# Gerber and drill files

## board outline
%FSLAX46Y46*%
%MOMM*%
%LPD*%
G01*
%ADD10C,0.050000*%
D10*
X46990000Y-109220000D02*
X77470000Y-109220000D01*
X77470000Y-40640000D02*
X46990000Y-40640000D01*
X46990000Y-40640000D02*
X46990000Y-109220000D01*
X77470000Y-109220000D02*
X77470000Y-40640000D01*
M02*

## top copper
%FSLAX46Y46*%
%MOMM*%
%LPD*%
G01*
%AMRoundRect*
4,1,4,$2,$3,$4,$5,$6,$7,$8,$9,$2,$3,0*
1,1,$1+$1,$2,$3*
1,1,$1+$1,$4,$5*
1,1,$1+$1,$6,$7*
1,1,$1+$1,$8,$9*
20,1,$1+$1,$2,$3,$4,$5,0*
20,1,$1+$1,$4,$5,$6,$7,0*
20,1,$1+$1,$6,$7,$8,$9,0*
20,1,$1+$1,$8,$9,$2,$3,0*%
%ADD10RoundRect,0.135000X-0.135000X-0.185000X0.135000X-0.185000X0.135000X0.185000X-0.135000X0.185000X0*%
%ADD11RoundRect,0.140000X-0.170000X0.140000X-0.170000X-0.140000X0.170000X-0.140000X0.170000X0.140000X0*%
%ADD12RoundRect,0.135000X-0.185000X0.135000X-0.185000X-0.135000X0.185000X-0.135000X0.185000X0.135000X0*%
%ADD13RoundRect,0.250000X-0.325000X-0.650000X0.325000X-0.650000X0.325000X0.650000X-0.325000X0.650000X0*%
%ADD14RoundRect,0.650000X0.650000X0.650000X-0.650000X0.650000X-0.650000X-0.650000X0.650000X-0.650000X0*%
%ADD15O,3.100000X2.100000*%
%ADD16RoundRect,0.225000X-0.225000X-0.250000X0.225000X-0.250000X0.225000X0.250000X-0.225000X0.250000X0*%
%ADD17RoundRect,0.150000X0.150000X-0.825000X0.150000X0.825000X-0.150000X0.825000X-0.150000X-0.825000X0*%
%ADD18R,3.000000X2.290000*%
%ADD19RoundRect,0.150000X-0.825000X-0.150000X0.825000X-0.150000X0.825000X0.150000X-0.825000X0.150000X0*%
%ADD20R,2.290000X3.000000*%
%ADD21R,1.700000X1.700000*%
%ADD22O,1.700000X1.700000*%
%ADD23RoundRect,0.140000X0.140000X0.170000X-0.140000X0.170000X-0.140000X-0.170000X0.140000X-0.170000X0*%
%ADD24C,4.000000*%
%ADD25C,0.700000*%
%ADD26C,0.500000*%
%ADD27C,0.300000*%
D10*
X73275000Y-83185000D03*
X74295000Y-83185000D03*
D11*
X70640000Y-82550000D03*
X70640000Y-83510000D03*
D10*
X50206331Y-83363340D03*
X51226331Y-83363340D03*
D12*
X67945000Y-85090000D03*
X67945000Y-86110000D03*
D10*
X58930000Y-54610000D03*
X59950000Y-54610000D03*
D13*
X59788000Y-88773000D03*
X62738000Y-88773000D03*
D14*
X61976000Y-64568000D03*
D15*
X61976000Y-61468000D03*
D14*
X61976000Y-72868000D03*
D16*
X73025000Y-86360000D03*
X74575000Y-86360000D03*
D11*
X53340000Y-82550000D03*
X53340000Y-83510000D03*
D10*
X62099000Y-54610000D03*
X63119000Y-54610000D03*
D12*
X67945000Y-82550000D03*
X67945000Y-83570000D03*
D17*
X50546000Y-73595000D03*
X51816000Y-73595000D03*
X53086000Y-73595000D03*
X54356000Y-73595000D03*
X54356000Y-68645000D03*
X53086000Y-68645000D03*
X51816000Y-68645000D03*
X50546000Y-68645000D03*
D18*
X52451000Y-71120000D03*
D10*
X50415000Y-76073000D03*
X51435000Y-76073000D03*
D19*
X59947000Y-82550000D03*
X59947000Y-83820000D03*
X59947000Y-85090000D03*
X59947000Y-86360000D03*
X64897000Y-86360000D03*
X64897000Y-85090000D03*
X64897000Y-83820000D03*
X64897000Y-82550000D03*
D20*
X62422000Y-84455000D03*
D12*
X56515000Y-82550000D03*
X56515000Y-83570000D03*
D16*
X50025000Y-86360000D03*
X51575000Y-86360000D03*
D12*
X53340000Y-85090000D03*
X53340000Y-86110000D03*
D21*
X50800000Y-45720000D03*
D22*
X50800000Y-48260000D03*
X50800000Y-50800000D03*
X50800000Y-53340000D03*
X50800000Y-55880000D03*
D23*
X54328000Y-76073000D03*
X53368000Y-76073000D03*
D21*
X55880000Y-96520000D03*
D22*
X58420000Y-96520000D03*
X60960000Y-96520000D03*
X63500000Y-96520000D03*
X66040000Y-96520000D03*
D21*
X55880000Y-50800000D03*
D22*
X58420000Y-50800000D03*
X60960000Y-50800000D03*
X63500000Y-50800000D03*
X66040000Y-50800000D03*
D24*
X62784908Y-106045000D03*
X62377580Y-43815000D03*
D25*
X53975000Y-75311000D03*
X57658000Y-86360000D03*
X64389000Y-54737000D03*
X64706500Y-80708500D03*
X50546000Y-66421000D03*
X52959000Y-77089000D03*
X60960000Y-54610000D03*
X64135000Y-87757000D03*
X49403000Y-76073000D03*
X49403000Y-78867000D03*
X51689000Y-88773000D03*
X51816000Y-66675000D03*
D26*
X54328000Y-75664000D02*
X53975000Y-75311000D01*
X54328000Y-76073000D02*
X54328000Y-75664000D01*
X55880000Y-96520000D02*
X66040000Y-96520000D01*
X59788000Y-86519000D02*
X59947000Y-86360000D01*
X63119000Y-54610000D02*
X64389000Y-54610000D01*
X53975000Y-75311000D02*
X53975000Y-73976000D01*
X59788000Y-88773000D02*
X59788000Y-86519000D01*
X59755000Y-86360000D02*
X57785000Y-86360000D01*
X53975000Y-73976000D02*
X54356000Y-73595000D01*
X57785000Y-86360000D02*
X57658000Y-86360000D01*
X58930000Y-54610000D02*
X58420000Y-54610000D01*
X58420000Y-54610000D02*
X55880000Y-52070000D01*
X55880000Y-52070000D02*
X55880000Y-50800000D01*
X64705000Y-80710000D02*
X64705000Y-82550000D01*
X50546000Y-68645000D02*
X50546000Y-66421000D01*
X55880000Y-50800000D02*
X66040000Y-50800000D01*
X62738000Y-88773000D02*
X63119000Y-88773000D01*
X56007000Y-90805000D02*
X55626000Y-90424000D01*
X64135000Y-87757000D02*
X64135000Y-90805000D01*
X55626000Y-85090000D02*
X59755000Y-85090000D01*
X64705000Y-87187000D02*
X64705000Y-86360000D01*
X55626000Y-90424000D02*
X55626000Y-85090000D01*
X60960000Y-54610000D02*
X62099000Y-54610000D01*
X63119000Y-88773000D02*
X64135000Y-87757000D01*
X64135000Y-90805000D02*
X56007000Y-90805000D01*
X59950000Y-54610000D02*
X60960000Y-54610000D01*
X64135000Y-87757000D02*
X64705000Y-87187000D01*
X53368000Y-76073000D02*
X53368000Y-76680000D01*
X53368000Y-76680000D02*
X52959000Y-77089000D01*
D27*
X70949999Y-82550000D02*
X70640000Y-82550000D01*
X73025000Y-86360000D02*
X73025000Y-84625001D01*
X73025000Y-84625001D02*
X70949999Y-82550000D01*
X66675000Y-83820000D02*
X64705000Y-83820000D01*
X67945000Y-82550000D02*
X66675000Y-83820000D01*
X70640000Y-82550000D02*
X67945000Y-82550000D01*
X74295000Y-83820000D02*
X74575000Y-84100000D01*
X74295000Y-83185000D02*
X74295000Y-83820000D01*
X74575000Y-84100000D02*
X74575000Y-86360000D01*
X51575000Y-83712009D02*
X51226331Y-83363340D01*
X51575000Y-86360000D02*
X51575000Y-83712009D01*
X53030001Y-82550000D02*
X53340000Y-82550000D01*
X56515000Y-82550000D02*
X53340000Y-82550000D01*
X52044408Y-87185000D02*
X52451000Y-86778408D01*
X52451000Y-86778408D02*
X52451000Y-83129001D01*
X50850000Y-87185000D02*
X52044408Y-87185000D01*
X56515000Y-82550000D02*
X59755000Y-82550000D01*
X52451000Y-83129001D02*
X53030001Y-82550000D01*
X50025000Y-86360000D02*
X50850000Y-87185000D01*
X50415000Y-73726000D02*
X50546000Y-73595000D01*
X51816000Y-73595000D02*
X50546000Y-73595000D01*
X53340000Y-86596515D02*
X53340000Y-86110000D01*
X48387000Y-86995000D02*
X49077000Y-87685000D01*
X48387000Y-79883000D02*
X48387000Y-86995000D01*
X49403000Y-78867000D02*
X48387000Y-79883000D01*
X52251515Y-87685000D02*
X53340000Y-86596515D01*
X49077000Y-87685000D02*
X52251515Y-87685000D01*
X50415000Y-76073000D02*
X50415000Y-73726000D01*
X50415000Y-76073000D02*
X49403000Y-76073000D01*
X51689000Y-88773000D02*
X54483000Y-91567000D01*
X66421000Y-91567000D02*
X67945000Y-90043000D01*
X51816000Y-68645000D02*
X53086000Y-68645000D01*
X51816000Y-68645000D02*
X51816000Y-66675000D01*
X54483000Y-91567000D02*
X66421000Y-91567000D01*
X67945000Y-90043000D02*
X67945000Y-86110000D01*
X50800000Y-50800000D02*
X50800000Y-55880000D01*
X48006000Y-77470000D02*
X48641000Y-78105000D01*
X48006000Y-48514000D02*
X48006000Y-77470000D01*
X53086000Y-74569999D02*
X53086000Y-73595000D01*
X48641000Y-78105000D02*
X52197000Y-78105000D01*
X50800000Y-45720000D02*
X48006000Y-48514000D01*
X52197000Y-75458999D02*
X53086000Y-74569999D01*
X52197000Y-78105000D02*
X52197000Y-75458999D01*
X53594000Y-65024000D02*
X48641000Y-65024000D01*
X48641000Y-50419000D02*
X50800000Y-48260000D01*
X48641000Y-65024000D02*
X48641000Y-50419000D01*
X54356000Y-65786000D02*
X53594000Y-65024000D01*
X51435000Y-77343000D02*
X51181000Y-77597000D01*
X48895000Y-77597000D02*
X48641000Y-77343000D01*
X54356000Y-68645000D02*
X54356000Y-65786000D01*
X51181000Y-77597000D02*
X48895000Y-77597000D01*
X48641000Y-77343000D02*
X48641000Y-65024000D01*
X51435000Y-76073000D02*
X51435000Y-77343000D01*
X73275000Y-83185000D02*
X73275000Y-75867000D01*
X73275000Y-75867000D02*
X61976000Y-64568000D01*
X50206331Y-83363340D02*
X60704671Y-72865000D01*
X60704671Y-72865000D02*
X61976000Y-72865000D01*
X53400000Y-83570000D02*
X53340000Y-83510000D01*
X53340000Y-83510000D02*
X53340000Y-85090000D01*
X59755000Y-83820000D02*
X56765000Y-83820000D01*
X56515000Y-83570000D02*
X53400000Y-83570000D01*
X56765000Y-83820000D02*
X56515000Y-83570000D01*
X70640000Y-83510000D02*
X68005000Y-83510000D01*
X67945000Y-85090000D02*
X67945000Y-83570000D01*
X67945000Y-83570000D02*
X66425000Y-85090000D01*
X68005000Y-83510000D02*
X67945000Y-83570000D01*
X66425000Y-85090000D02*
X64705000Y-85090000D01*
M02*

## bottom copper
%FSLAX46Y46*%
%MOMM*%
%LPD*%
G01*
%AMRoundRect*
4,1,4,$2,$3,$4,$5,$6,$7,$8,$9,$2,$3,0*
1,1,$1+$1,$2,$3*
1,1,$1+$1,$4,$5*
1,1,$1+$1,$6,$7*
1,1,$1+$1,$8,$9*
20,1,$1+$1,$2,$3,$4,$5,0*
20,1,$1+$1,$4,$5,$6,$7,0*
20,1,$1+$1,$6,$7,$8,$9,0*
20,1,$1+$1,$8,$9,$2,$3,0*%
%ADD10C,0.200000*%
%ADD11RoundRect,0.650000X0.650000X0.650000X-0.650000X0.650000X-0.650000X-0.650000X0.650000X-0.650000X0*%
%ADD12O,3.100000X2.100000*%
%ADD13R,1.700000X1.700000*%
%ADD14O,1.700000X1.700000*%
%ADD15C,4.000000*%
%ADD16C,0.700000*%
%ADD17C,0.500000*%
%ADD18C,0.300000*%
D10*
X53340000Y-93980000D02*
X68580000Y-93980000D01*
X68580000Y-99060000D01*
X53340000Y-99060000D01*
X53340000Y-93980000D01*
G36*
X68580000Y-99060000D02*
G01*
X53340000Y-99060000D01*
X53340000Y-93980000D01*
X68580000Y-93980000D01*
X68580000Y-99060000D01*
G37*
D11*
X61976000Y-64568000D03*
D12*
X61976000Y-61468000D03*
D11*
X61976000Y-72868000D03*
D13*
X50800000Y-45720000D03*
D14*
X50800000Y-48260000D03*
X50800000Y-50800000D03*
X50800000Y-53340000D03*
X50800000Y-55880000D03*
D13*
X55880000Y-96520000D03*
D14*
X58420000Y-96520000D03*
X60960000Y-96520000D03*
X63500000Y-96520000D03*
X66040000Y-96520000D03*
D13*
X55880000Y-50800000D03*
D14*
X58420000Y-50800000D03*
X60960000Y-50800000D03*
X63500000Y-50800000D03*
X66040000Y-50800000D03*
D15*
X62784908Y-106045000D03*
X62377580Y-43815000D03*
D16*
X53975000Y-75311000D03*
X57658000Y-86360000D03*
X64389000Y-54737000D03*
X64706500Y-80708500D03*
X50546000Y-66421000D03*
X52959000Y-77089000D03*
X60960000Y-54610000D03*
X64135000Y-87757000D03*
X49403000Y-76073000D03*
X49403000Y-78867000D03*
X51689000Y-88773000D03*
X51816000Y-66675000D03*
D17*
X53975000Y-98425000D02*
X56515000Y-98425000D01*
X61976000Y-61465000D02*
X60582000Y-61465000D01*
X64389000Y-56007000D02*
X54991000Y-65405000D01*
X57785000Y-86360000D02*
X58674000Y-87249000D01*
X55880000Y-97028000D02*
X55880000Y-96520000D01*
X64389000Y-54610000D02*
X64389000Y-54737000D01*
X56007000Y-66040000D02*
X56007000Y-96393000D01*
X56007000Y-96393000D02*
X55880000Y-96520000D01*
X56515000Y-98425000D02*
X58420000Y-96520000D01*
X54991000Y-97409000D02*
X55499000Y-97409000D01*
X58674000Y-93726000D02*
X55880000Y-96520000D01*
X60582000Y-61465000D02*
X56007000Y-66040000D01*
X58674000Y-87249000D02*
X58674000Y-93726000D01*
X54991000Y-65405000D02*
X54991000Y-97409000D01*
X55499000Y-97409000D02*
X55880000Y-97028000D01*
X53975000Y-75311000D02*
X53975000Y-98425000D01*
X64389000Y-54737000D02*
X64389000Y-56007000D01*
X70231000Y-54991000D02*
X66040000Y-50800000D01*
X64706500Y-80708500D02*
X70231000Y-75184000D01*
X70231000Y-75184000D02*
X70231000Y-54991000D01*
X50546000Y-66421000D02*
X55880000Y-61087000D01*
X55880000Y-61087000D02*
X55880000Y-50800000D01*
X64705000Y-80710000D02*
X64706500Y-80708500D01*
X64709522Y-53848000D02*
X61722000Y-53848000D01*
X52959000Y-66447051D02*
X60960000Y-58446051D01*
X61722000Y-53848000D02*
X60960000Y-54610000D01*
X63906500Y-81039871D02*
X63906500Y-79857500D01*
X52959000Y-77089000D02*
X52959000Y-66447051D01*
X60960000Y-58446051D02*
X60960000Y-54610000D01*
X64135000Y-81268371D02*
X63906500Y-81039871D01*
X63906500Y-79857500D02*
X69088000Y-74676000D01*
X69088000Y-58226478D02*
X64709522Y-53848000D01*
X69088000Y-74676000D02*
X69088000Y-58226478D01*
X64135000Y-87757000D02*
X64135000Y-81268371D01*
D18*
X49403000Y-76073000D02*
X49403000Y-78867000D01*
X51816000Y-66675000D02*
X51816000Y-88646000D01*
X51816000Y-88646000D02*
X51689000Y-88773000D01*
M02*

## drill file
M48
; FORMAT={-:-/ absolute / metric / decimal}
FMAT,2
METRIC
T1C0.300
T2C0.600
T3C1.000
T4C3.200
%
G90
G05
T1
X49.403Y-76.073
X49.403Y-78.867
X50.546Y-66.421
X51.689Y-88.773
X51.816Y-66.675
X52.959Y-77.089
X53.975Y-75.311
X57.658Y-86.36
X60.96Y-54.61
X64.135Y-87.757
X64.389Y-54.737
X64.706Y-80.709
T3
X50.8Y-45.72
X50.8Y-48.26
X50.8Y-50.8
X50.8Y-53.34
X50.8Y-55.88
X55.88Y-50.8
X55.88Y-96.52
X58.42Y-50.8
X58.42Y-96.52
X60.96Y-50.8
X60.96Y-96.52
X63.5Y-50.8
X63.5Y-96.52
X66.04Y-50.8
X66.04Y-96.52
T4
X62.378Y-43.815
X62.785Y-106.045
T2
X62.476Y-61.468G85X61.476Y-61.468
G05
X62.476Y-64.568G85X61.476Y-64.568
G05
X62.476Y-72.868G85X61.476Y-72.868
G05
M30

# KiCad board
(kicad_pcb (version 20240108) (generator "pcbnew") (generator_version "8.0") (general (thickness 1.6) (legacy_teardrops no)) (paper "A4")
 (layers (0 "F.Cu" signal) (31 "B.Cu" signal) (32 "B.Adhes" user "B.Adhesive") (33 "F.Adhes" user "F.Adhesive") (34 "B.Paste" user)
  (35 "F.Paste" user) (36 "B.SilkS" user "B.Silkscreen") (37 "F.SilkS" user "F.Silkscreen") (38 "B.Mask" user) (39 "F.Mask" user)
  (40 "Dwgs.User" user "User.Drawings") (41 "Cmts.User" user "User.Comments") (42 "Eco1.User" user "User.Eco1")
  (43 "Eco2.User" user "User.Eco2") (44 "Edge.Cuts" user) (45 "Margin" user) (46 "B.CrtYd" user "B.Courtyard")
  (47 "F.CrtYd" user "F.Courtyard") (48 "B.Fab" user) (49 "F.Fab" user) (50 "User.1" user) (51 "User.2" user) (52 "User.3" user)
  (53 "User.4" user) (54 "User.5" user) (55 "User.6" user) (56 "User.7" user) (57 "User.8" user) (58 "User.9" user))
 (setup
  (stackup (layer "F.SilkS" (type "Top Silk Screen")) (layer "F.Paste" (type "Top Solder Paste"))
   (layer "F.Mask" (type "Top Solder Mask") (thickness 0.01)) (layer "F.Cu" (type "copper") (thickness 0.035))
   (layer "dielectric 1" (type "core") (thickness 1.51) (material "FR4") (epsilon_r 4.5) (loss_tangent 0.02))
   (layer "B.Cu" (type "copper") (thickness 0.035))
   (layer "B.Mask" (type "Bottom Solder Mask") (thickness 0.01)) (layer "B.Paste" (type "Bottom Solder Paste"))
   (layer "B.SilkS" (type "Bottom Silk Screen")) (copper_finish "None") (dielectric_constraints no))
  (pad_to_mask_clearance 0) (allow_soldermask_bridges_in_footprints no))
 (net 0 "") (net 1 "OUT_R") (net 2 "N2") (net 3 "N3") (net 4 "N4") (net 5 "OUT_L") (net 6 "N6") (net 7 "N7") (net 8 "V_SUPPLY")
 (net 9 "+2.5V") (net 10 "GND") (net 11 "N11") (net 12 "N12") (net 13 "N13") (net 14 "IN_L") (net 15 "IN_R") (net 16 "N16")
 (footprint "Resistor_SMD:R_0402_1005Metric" (layer "F.Cu") (at 73.785 83.185)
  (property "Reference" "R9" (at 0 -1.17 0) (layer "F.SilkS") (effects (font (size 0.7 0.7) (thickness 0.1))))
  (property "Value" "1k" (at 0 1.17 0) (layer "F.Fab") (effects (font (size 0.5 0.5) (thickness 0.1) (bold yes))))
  (pad "1" smd roundrect (at -0.51 0) (size 0.54 0.64) (layers "F.Cu" "F.Paste" "F.Mask") (roundrect_rratio 0.25) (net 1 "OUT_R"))
  (pad "2" smd roundrect (at 0.51 0) (size 0.54 0.64) (layers "F.Cu" "F.Paste" "F.Mask") (roundrect_rratio 0.25) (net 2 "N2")))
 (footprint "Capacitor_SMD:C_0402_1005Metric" (layer "F.Cu") (at 70.64 83.03 -90)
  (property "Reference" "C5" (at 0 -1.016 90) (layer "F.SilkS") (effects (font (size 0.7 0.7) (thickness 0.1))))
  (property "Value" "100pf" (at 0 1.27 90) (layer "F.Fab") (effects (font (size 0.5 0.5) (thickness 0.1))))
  (pad "1" smd roundrect (at -0.48 0 270) (size 0.56 0.62) (layers "F.Cu" "F.Paste" "F.Mask") (roundrect_rratio 0.25) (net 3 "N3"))
  (pad "2" smd roundrect (at 0.48 0 270) (size 0.56 0.62) (layers "F.Cu" "F.Paste" "F.Mask") (roundrect_rratio 0.25) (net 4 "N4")))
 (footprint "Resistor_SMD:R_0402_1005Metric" (layer "F.Cu") (at 50.716331 83.36334)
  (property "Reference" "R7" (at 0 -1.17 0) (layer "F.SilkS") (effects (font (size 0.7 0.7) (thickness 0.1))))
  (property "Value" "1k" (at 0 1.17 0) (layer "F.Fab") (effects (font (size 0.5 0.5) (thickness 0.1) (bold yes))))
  (pad "1" smd roundrect (at -0.51 0) (size 0.54 0.64) (layers "F.Cu" "F.Paste" "F.Mask") (roundrect_rratio 0.25) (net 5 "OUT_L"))
  (pad "2" smd roundrect (at 0.51 0) (size 0.54 0.64) (layers "F.Cu" "F.Paste" "F.Mask") (roundrect_rratio 0.25) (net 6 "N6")))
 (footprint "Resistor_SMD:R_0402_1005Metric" (layer "F.Cu") (at 67.945 85.6 -90)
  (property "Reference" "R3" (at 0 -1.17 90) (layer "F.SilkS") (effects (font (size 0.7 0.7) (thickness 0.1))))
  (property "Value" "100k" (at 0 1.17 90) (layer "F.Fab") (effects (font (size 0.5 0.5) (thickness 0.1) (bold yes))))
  (pad "1" smd roundrect (at -0.51 0 270) (size 0.54 0.64) (layers "F.Cu" "F.Paste" "F.Mask") (roundrect_rratio 0.25) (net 4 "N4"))
  (pad "2" smd roundrect (at 0.51 0 270) (size 0.54 0.64) (layers "F.Cu" "F.Paste" "F.Mask") (roundrect_rratio 0.25) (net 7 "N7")))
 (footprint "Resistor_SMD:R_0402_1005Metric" (layer "F.Cu") (at 59.44 54.61)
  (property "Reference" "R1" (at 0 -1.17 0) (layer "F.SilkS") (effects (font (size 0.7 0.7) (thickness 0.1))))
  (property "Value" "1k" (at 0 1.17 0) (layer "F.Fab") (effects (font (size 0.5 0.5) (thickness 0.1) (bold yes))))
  (pad "1" smd roundrect (at -0.51 0) (size 0.54 0.64) (layers "F.Cu" "F.Paste" "F.Mask") (roundrect_rratio 0.25) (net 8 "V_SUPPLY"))
  (pad "2" smd roundrect (at 0.51 0) (size 0.54 0.64) (layers "F.Cu" "F.Paste" "F.Mask") (roundrect_rratio 0.25) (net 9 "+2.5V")))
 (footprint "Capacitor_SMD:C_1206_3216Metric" (layer "F.Cu") (at 61.263 88.773)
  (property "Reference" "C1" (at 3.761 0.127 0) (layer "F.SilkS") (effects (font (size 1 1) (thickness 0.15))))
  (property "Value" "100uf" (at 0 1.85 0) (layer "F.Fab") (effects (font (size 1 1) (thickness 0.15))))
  (pad "1" smd roundrect (at -1.475 0) (size 1.15 1.8) (layers "F.Cu" "F.Paste" "F.Mask") (roundrect_rratio 0.217391) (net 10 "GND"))
  (pad "2" smd roundrect (at 1.475 0) (size 1.15 1.8) (layers "F.Cu" "F.Paste" "F.Mask") (roundrect_rratio 0.217391) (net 9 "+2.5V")))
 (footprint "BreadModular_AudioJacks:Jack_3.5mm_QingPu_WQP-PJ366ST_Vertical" (layer "F.Cu") (at 61.976 67.948 180)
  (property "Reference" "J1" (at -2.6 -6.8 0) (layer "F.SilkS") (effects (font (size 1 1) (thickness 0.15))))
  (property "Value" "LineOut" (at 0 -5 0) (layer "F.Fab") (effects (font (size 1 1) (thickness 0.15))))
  (pad "R" thru_hole roundrect (at 0 3.38 180) (size 2.6 2.6) (drill oval 1.6 0.6) (layers "*.Cu" "*.Mask") (remove_unused_layers no)
   (roundrect_rratio 0.25) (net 1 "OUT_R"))
  (pad "S" thru_hole oval (at 0 6.48 180) (size 3.1 2.1) (drill oval 1.6 0.6) (layers "*.Cu" "*.Mask") (remove_unused_layers no)
   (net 10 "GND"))
  (pad "T" thru_hole roundrect (at 0 -4.92 180) (size 2.6 2.6) (drill oval 1.6 0.6) (layers "*.Cu" "*.Mask") (remove_unused_layers no)
   (roundrect_rratio 0.25) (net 5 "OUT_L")))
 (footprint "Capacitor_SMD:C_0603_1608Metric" (layer "F.Cu") (at 73.8 86.36)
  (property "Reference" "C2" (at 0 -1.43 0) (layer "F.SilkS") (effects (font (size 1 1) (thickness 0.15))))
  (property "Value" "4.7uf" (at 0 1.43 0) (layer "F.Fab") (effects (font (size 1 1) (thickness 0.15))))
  (pad "1" smd roundrect (at -0.775 0) (size 0.9 0.95) (layers "F.Cu" "F.Paste" "F.Mask") (roundrect_rratio 0.25) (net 3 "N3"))
  (pad "2" smd roundrect (at 0.775 0) (size 0.9 0.95) (layers "F.Cu" "F.Paste" "F.Mask") (roundrect_rratio 0.25) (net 2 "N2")))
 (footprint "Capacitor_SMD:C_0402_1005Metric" (layer "F.Cu") (at 53.34 83.03 -90)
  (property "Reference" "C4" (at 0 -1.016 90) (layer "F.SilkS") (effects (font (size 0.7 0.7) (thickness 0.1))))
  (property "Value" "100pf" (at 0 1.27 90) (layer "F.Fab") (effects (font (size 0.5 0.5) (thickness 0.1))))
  (pad "1" smd roundrect (at -0.48 0 270) (size 0.56 0.62) (layers "F.Cu" "F.Paste" "F.Mask") (roundrect_rratio 0.25) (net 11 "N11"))
  (pad "2" smd roundrect (at 0.48 0 270) (size 0.56 0.62) (layers "F.Cu" "F.Paste" "F.Mask") (roundrect_rratio 0.25) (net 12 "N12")))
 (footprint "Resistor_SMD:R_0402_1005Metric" (layer "F.Cu") (at 62.609 54.61)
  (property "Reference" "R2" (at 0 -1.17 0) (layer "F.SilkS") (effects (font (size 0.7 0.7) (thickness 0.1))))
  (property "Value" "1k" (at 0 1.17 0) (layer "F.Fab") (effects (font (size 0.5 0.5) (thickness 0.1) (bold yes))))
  (pad "1" smd roundrect (at -0.51 0) (size 0.54 0.64) (layers "F.Cu" "F.Paste" "F.Mask") (roundrect_rratio 0.25) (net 9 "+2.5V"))
  (pad "2" smd roundrect (at 0.51 0) (size 0.54 0.64) (layers "F.Cu" "F.Paste" "F.Mask") (roundrect_rratio 0.25) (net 10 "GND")))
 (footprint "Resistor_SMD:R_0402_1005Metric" (layer "F.Cu") (at 67.945 83.06 -90)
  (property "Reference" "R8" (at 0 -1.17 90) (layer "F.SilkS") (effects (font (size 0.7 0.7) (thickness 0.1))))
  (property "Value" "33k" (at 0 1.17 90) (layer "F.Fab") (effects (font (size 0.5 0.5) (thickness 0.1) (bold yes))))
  (pad "1" smd roundrect (at -0.51 0 270) (size 0.54 0.64) (layers "F.Cu" "F.Paste" "F.Mask") (roundrect_rratio 0.25) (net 3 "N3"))
  (pad "2" smd roundrect (at 0.51 0 270) (size 0.54 0.64) (layers "F.Cu" "F.Paste" "F.Mask") (roundrect_rratio 0.25) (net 4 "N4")))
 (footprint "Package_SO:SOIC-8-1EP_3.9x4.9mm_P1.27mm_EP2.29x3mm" (layer "F.Cu") (at 52.451 71.12 90)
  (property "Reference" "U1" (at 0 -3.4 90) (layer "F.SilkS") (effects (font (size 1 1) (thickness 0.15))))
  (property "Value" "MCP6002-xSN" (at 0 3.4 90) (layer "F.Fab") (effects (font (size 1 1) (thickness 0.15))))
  (pad "" smd roundrect (at -0.57 -0.75 90) (size 0.92 1.21) (layers "F.Paste") (roundrect_rratio 0.25))
  (pad "" smd roundrect (at -0.57 0.75 90) (size 0.92 1.21) (layers "F.Paste") (roundrect_rratio 0.25))
  (pad "" smd roundrect (at 0.57 -0.75 90) (size 0.92 1.21) (layers "F.Paste") (roundrect_rratio 0.25))
  (pad "" smd roundrect (at 0.57 0.75 90) (size 0.92 1.21) (layers "F.Paste") (roundrect_rratio 0.25))
  (pad "1" smd roundrect (at -2.475 -1.905 90) (size 1.95 0.6) (layers "F.Cu" "F.Paste" "F.Mask") (roundrect_rratio 0.25) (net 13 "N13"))
  (pad "2" smd roundrect (at -2.475 -0.635 90) (size 1.95 0.6) (layers "F.Cu" "F.Paste" "F.Mask") (roundrect_rratio 0.25) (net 13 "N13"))
  (pad "3" smd roundrect (at -2.475 0.635 90) (size 1.95 0.6) (layers "F.Cu" "F.Paste" "F.Mask") (roundrect_rratio 0.25) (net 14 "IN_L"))
  (pad "4" smd roundrect (at -2.475 1.905 90) (size 1.95 0.6) (layers "F.Cu" "F.Paste" "F.Mask") (roundrect_rratio 0.25) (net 10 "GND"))
  (pad "5" smd roundrect (at 2.475 1.905 90) (size 1.95 0.6) (layers "F.Cu" "F.Paste" "F.Mask") (roundrect_rratio 0.25) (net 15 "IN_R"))
  (pad "6" smd roundrect (at 2.475 0.635 90) (size 1.95 0.6) (layers "F.Cu" "F.Paste" "F.Mask") (roundrect_rratio 0.25) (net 7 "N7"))
  (pad "7" smd roundrect (at 2.475 -0.635 90) (size 1.95 0.6) (layers "F.Cu" "F.Paste" "F.Mask") (roundrect_rratio 0.25) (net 7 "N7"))
  (pad "8" smd roundrect (at 2.475 -1.905 90) (size 1.95 0.6) (layers "F.Cu" "F.Paste" "F.Mask") (roundrect_rratio 0.25) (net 8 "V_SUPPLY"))
  (pad "9" smd rect (at 0 0 90) (size 2.29 3) (layers "F.Cu" "F.Mask") (zone_connect 2)))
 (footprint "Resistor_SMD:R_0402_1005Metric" (layer "F.Cu") (at 50.925 76.073)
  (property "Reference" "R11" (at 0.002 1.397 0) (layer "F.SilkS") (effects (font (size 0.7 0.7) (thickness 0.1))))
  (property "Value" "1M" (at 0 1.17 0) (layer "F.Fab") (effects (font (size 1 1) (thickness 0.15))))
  (pad "1" smd roundrect (at -0.51 0) (size 0.54 0.64) (layers "F.Cu" "F.Paste" "F.Mask") (roundrect_rratio 0.25) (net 13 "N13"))
  (pad "2" smd roundrect (at 0.51 0) (size 0.54 0.64) (layers "F.Cu" "F.Paste" "F.Mask") (roundrect_rratio 0.25) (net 15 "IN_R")))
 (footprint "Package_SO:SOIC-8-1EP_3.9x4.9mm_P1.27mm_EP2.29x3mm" (layer "F.Cu") (at 62.422 84.455)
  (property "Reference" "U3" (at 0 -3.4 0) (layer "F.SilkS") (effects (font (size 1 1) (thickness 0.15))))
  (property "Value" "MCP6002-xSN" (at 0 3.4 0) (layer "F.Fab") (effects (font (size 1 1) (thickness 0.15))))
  (pad "" smd roundrect (at -0.57 -0.75) (size 0.92 1.21) (layers "F.Paste") (roundrect_rratio 0.25))
  (pad "" smd roundrect (at -0.57 0.75) (size 0.92 1.21) (layers "F.Paste") (roundrect_rratio 0.25))
  (pad "" smd roundrect (at 0.57 -0.75) (size 0.92 1.21) (layers "F.Paste") (roundrect_rratio 0.25))
  (pad "" smd roundrect (at 0.57 0.75) (size 0.92 1.21) (layers "F.Paste") (roundrect_rratio 0.25))
  (pad "1" smd roundrect (at -2.475 -1.905) (size 1.95 0.6) (layers "F.Cu" "F.Paste" "F.Mask") (roundrect_rratio 0.25) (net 11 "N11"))
  (pad "2" smd roundrect (at -2.475 -0.635) (size 1.95 0.6) (layers "F.Cu" "F.Paste" "F.Mask") (roundrect_rratio 0.25) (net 12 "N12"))
  (pad "3" smd roundrect (at -2.475 0.635) (size 1.95 0.6) (layers "F.Cu" "F.Paste" "F.Mask") (roundrect_rratio 0.25) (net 9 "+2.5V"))
  (pad "4" smd roundrect (at -2.475 1.905) (size 1.95 0.6) (layers "F.Cu" "F.Paste" "F.Mask") (roundrect_rratio 0.25) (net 10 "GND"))
  (pad "5" smd roundrect (at 2.475 1.905) (size 1.95 0.6) (layers "F.Cu" "F.Paste" "F.Mask") (roundrect_rratio 0.25) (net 9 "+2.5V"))
  (pad "6" smd roundrect (at 2.475 0.635) (size 1.95 0.6) (layers "F.Cu" "F.Paste" "F.Mask") (roundrect_rratio 0.25) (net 4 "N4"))
  (pad "7" smd roundrect (at 2.475 -0.635) (size 1.95 0.6) (layers "F.Cu" "F.Paste" "F.Mask") (roundrect_rratio 0.25) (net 3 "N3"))
  (pad "8" smd roundrect (at 2.475 -1.905) (size 1.95 0.6) (layers "F.Cu" "F.Paste" "F.Mask") (roundrect_rratio 0.25) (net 8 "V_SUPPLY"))
  (pad "9" smd rect (at 0 0) (size 2.29 3) (layers "F.Cu" "F.Mask") (zone_connect 2)))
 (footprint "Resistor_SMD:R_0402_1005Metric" (layer "F.Cu") (at 56.515 83.06 -90)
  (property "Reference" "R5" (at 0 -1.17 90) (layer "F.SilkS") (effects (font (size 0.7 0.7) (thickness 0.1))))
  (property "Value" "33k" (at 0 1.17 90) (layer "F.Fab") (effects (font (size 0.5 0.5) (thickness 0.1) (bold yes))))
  (pad "1" smd roundrect (at -0.51 0 270) (size 0.54 0.64) (layers "F.Cu" "F.Paste" "F.Mask") (roundrect_rratio 0.25) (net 11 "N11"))
  (pad "2" smd roundrect (at 0.51 0 270) (size 0.54 0.64) (layers "F.Cu" "F.Paste" "F.Mask") (roundrect_rratio 0.25) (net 12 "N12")))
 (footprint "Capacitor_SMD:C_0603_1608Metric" (layer "F.Cu") (at 50.8 86.36)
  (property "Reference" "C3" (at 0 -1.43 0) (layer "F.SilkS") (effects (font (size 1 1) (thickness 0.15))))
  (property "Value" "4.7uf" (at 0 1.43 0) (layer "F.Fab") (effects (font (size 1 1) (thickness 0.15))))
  (pad "1" smd roundrect (at -0.775 0) (size 0.9 0.95) (layers "F.Cu" "F.Paste" "F.Mask") (roundrect_rratio 0.25) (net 11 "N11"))
  (pad "2" smd roundrect (at 0.775 0) (size 0.9 0.95) (layers "F.Cu" "F.Paste" "F.Mask") (roundrect_rratio 0.25) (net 6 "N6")))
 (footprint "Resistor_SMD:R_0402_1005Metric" (layer "F.Cu") (at 53.34 85.6 -90)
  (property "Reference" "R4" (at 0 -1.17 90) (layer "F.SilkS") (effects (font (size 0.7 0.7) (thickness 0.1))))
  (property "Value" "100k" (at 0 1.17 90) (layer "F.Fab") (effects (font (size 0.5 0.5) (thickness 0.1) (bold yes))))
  (pad "1" smd roundrect (at -0.51 0 270) (size 0.54 0.64) (layers "F.Cu" "F.Paste" "F.Mask") (roundrect_rratio 0.25) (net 12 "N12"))
  (pad "2" smd roundrect (at 0.51 0 270) (size 0.54 0.64) (layers "F.Cu" "F.Paste" "F.Mask") (roundrect_rratio 0.25) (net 13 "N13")))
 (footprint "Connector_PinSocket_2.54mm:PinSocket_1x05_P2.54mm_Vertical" (layer "F.Cu") (at 50.8 45.72)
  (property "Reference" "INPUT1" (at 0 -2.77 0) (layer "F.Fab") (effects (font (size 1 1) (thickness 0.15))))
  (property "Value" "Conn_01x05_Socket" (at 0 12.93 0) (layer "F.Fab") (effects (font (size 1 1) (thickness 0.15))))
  (pad "1" thru_hole rect (at 0 0) (size 1.7 1.7) (drill 1) (layers "*.Cu" "*.Mask") (remove_unused_layers no) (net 14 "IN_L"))
  (pad "2" thru_hole oval (at 0 2.54) (size 1.7 1.7) (drill 1) (layers "*.Cu" "*.Mask") (remove_unused_layers no) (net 15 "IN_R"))
  (pad "3" thru_hole oval (at 0 5.08) (size 1.7 1.7) (drill 1) (layers "*.Cu" "*.Mask") (remove_unused_layers no) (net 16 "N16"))
  (pad "4" thru_hole oval (at 0 7.62) (size 1.7 1.7) (drill 1) (layers "*.Cu" "*.Mask") (remove_unused_layers no) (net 16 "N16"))
  (pad "5" thru_hole oval (at 0 10.16) (size 1.7 1.7) (drill 1) (layers "*.Cu" "*.Mask") (remove_unused_layers no) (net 16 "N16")))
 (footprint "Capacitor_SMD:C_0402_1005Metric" (layer "F.Cu") (at 53.848 76.073 180)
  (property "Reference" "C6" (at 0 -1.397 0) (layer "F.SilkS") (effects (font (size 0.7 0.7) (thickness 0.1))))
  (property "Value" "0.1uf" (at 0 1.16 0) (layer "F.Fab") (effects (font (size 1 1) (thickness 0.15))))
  (pad "1" smd roundrect (at -0.48 0 180) (size 0.56 0.62) (layers "F.Cu" "F.Paste" "F.Mask") (roundrect_rratio 0.25) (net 10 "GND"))
  (pad "2" smd roundrect (at 0.48 0 180) (size 0.56 0.62) (layers "F.Cu" "F.Paste" "F.Mask") (roundrect_rratio 0.25) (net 9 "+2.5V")))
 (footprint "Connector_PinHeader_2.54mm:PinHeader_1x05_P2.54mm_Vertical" (layer "B.Cu") (at 55.88 96.52 -90)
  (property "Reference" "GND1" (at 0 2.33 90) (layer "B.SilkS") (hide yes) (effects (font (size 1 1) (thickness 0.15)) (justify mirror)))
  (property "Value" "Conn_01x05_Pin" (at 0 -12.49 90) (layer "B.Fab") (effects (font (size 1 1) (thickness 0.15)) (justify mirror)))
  (pad "1" thru_hole rect (at 0 0 270) (size 1.7 1.7) (drill 1) (layers "*.Cu" "*.Mask") (remove_unused_layers no) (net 10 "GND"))
  (pad "2" thru_hole oval (at 0 -2.54 270) (size 1.7 1.7) (drill 1) (layers "*.Cu" "*.Mask") (remove_unused_layers no) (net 10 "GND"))
  (pad "3" thru_hole oval (at 0 -5.08 270) (size 1.7 1.7) (drill 1) (layers "*.Cu" "*.Mask") (remove_unused_layers no) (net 10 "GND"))
  (pad "4" thru_hole oval (at 0 -7.62 270) (size 1.7 1.7) (drill 1) (layers "*.Cu" "*.Mask") (remove_unused_layers no) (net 10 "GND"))
  (pad "5" thru_hole oval (at 0 -10.16 270) (size 1.7 1.7) (drill 1) (layers "*.Cu" "*.Mask") (remove_unused_layers no) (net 10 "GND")))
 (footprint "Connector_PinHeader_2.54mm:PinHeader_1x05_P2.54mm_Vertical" (layer "B.Cu") (at 55.88 50.8 -90)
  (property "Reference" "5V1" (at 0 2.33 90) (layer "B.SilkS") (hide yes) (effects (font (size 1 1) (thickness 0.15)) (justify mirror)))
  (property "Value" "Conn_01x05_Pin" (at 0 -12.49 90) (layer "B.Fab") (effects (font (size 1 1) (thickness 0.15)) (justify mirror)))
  (pad "1" thru_hole rect (at 0 0 270) (size 1.7 1.7) (drill 1) (layers "*.Cu" "*.Mask") (remove_unused_layers no) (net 8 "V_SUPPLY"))
  (pad "2" thru_hole oval (at 0 -2.54 270) (size 1.7 1.7) (drill 1) (layers "*.Cu" "*.Mask") (remove_unused_layers no) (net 8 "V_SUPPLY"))
  (pad "3" thru_hole oval (at 0 -5.08 270) (size 1.7 1.7) (drill 1) (layers "*.Cu" "*.Mask") (remove_unused_layers no) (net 8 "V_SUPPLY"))
  (pad "4" thru_hole oval (at 0 -7.62 270) (size 1.7 1.7) (drill 1) (layers "*.Cu" "*.Mask") (remove_unused_layers no) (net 8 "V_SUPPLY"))
  (pad "5" thru_hole oval (at 0 -10.16 270) (size 1.7 1.7) (drill 1) (layers "*.Cu" "*.Mask") (remove_unused_layers no) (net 8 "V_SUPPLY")))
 (gr_poly
  (pts (xy 53.34 93.98) (xy 68.58 93.98) (xy 68.58 99.06) (xy 53.34 99.06)) (stroke (width 0.2) (type solid)) (fill solid) (layer "B.Cu")
  (net 10))
 (gr_line (start 46.99 109.22) (end 77.47 109.22) (stroke (width 0.05) (type default)) (layer "Edge.Cuts"))
 (gr_line (start 77.47 40.64) (end 46.99 40.64) (stroke (width 0.05) (type default)) (layer "Edge.Cuts"))
 (gr_line (start 46.99 40.64) (end 46.99 109.22) (stroke (width 0.05) (type default)) (layer "Edge.Cuts"))
 (gr_line (start 77.47 109.22) (end 77.47 40.64) (stroke (width 0.05) (type default)) (layer "Edge.Cuts"))
 (via (at 62.784908 106.045) (size 4) (drill 3.2) (layers "F.Cu" "B.Cu") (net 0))
 (via (at 62.37758 43.815) (size 4) (drill 3.2) (layers "F.Cu" "B.Cu") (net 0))
 (segment (start 54.328 75.664) (end 53.975 75.311) (width 0.5) (layer "F.Cu") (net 10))
 (segment (start 54.328 76.073) (end 54.328 75.664) (width 0.5) (layer "F.Cu") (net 10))
 (segment (start 55.88 96.52) (end 66.04 96.52) (width 0.5) (layer "F.Cu") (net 10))
 (segment (start 59.788 86.519) (end 59.947 86.36) (width 0.5) (layer "F.Cu") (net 10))
 (segment (start 63.119 54.61) (end 64.389 54.61) (width 0.5) (layer "F.Cu") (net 10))
 (segment (start 53.975 75.311) (end 53.975 73.976) (width 0.5) (layer "F.Cu") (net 10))
 (segment (start 59.788 88.773) (end 59.788 86.519) (width 0.5) (layer "F.Cu") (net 10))
 (segment (start 59.755 86.36) (end 57.785 86.36) (width 0.5) (layer "F.Cu") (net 10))
 (segment (start 53.975 73.976) (end 54.356 73.595) (width 0.5) (layer "F.Cu") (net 10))
 (segment (start 57.785 86.36) (end 57.658 86.36) (width 0.5) (layer "F.Cu") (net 10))
 (via (at 53.975 75.311) (size 0.7) (drill 0.3) (layers "F.Cu" "B.Cu") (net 10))
 (via (at 57.658 86.36) (size 0.7) (drill 0.3) (layers "F.Cu" "B.Cu") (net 10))
 (via (at 64.389 54.737) (size 0.7) (drill 0.3) (layers "F.Cu" "B.Cu") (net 10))
 (segment (start 53.975 98.425) (end 56.515 98.425) (width 0.5) (layer "B.Cu") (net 10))
 (segment (start 61.976 61.465) (end 60.582 61.465) (width 0.5) (layer "B.Cu") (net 10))
 (segment (start 64.389 56.007) (end 54.991 65.405) (width 0.5) (layer "B.Cu") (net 10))
 (segment (start 57.785 86.36) (end 58.674 87.249) (width 0.5) (layer "B.Cu") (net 10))
 (segment (start 55.88 97.028) (end 55.88 96.52) (width 0.5) (layer "B.Cu") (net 10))
 (segment (start 64.389 54.61) (end 64.389 54.737) (width 0.5) (layer "B.Cu") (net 10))
 (segment (start 56.007 66.04) (end 56.007 96.393) (width 0.5) (layer "B.Cu") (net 10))
 (segment (start 56.007 96.393) (end 55.88 96.52) (width 0.5) (layer "B.Cu") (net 10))
 (segment (start 56.515 98.425) (end 58.42 96.52) (width 0.5) (layer "B.Cu") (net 10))
 (segment (start 54.991 97.409) (end 55.499 97.409) (width 0.5) (layer "B.Cu") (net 10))
 (segment (start 58.674 93.726) (end 55.88 96.52) (width 0.5) (layer "B.Cu") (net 10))
 (segment (start 60.582 61.465) (end 56.007 66.04) (width 0.5) (layer "B.Cu") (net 10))
 (segment (start 58.674 87.249) (end 58.674 93.726) (width 0.5) (layer "B.Cu") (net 10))
 (segment (start 54.991 65.405) (end 54.991 97.409) (width 0.5) (layer "B.Cu") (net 10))
 (segment (start 55.499 97.409) (end 55.88 97.028) (width 0.5) (layer "B.Cu") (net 10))
 (segment (start 53.975 75.311) (end 53.975 98.425) (width 0.5) (layer "B.Cu") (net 10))
 (segment (start 64.389 54.737) (end 64.389 56.007) (width 0.5) (layer "B.Cu") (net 10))
 (segment (start 58.93 54.61) (end 58.42 54.61) (width 0.5) (layer "F.Cu") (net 8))
 (segment (start 58.42 54.61) (end 55.88 52.07) (width 0.5) (layer "F.Cu") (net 8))
 (segment (start 55.88 52.07) (end 55.88 50.8) (width 0.5) (layer "F.Cu") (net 8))
 (segment (start 64.705 80.71) (end 64.705 82.55) (width 0.5) (layer "F.Cu") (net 8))
 (segment (start 50.546 68.645) (end 50.546 66.421) (width 0.5) (layer "F.Cu") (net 8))
 (segment (start 55.88 50.8) (end 66.04 50.8) (width 0.5) (layer "F.Cu") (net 8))
 (via (at 64.7065 80.7085) (size 0.7) (drill 0.3) (layers "F.Cu" "B.Cu") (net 8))
 (via (at 50.546 66.421) (size 0.7) (drill 0.3) (layers "F.Cu" "B.Cu") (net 8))
 (segment (start 70.231 54.991) (end 66.04 50.8) (width 0.5) (layer "B.Cu") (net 8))
 (segment (start 64.7065 80.7085) (end 70.231 75.184) (width 0.5) (layer "B.Cu") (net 8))
 (segment (start 70.231 75.184) (end 70.231 54.991) (width 0.5) (layer "B.Cu") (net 8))
 (segment (start 50.546 66.421) (end 55.88 61.087) (width 0.5) (layer "B.Cu") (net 8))
 (segment (start 55.88 61.087) (end 55.88 50.8) (width 0.5) (layer "B.Cu") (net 8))
 (segment (start 64.705 80.71) (end 64.7065 80.7085) (width 0.5) (layer "B.Cu") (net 8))
 (segment (start 62.738 88.773) (end 63.119 88.773) (width 0.5) (layer "F.Cu") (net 9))
 (segment (start 56.007 90.805) (end 55.626 90.424) (width 0.5) (layer "F.Cu") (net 9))
 (segment (start 64.135 87.757) (end 64.135 90.805) (width 0.5) (layer "F.Cu") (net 9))
 (segment (start 55.626 85.09) (end 59.755 85.09) (width 0.5) (layer "F.Cu") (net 9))
 (segment (start 64.705 87.187) (end 64.705 86.36) (width 0.5) (layer "F.Cu") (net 9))
 (segment (start 55.626 90.424) (end 55.626 85.09) (width 0.5) (layer "F.Cu") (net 9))
 (segment (start 60.96 54.61) (end 62.099 54.61) (width 0.5) (layer "F.Cu") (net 9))
 (segment (start 63.119 88.773) (end 64.135 87.757) (width 0.5) (layer "F.Cu") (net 9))
 (segment (start 64.135 90.805) (end 56.007 90.805) (width 0.5) (layer "F.Cu") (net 9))
 (segment (start 59.95 54.61) (end 60.96 54.61) (width 0.5) (layer "F.Cu") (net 9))
 (segment (start 64.135 87.757) (end 64.705 87.187) (width 0.5) (layer "F.Cu") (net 9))
 (segment (start 53.368 76.073) (end 53.368 76.68) (width 0.5) (layer "F.Cu") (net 9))
 (segment (start 53.368 76.68) (end 52.959 77.089) (width 0.5) (layer "F.Cu") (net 9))
 (via (at 52.959 77.089) (size 0.7) (drill 0.3) (layers "F.Cu" "B.Cu") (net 9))
 (via (at 60.96 54.61) (size 0.7) (drill 0.3) (layers "F.Cu" "B.Cu") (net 9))
 (via (at 64.135 87.757) (size 0.7) (drill 0.3) (layers "F.Cu" "B.Cu") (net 9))
 (segment (start 64.709522 53.848) (end 61.722 53.848) (width 0.5) (layer "B.Cu") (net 9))
 (segment (start 52.959 66.447051) (end 60.96 58.446051) (width 0.5) (layer "B.Cu") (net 9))
 (segment (start 61.722 53.848) (end 60.96 54.61) (width 0.5) (layer "B.Cu") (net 9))
 (segment (start 63.9065 81.039871) (end 63.9065 79.8575) (width 0.5) (layer "B.Cu") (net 9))
 (segment (start 52.959 77.089) (end 52.959 66.447051) (width 0.5) (layer "B.Cu") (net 9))
 (segment (start 60.96 58.446051) (end 60.96 54.61) (width 0.5) (layer "B.Cu") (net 9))
 (segment (start 64.135 81.268371) (end 63.9065 81.039871) (width 0.5) (layer "B.Cu") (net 9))
 (segment (start 63.9065 79.8575) (end 69.088 74.676) (width 0.5) (layer "B.Cu") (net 9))
 (segment (start 69.088 58.226478) (end 64.709522 53.848) (width 0.5) (layer "B.Cu") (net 9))
 (segment (start 69.088 74.676) (end 69.088 58.226478) (width 0.5) (layer "B.Cu") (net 9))
 (segment (start 64.135 87.757) (end 64.135 81.268371) (width 0.5) (layer "B.Cu") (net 9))
 (segment (start 70.949999 82.55) (end 70.64 82.55) (width 0.3) (layer "F.Cu") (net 3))
 (segment (start 73.025 86.36) (end 73.025 84.625001) (width 0.3) (layer "F.Cu") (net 3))
 (segment (start 73.025 84.625001) (end 70.949999 82.55) (width 0.3) (layer "F.Cu") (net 3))
 (segment (start 66.675 83.82) (end 64.705 83.82) (width 0.3) (layer "F.Cu") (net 3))
 (segment (start 67.945 82.55) (end 66.675 83.82) (width 0.3) (layer "F.Cu") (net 3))
 (segment (start 70.64 82.55) (end 67.945 82.55) (width 0.3) (layer "F.Cu") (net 3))
 (segment (start 74.295 83.82) (end 74.575 84.1) (width 0.3) (layer "F.Cu") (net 2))
 (segment (start 74.295 83.185) (end 74.295 83.82) (width 0.3) (layer "F.Cu") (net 2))
 (segment (start 74.575 84.1) (end 74.575 86.36) (width 0.3) (layer "F.Cu") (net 2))
 (segment (start 51.575 83.712009) (end 51.226331 83.36334) (width 0.3) (layer "F.Cu") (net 6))
 (segment (start 51.575 86.36) (end 51.575 83.712009) (width 0.3) (layer "F.Cu") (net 6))
 (segment (start 53.030001 82.55) (end 53.34 82.55) (width 0.3) (layer "F.Cu") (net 11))
 (segment (start 56.515 82.55) (end 53.34 82.55) (width 0.3) (layer "F.Cu") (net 11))
 (segment (start 52.044408 87.185) (end 52.451 86.778408) (width 0.3) (layer "F.Cu") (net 11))
 (segment (start 52.451 86.778408) (end 52.451 83.129001) (width 0.3) (layer "F.Cu") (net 11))
 (segment (start 50.85 87.185) (end 52.044408 87.185) (width 0.3) (layer "F.Cu") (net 11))
 (segment (start 56.515 82.55) (end 59.755 82.55) (width 0.3) (layer "F.Cu") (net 11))
 (segment (start 52.451 83.129001) (end 53.030001 82.55) (width 0.3) (layer "F.Cu") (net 11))
 (segment (start 50.025 86.36) (end 50.85 87.185) (width 0.3) (layer "F.Cu") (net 11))
 (segment (start 50.415 73.726) (end 50.546 73.595) (width 0.3) (layer "F.Cu") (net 13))
 (segment (start 51.816 73.595) (end 50.546 73.595) (width 0.3) (layer "F.Cu") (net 13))
 (segment (start 53.34 86.596515) (end 53.34 86.11) (width 0.3) (layer "F.Cu") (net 13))
 (segment (start 48.387 86.995) (end 49.077 87.685) (width 0.3) (layer "F.Cu") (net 13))
 (segment (start 48.387 79.883) (end 48.387 86.995) (width 0.3) (layer "F.Cu") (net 13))
 (segment (start 49.403 78.867) (end 48.387 79.883) (width 0.3) (layer "F.Cu") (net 13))
 (segment (start 52.251515 87.685) (end 53.34 86.596515) (width 0.3) (layer "F.Cu") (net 13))
 (segment (start 49.077 87.685) (end 52.251515 87.685) (width 0.3) (layer "F.Cu") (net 13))
 (segment (start 50.415 76.073) (end 50.415 73.726) (width 0.3) (layer "F.Cu") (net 13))
 (segment (start 50.415 76.073) (end 49.403 76.073) (width 0.3) (layer "F.Cu") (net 13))
 (via (at 49.403 76.073) (size 0.7) (drill 0.3) (layers "F.Cu" "B.Cu") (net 13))
 (via (at 49.403 78.867) (size 0.7) (drill 0.3) (layers "F.Cu" "B.Cu") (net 13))
 (segment (start 49.403 76.073) (end 49.403 78.867) (width 0.3) (layer "B.Cu") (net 13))
 (segment (start 51.689 88.773) (end 54.483 91.567) (width 0.3) (layer "F.Cu") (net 7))
 (segment (start 66.421 91.567) (end 67.945 90.043) (width 0.3) (layer "F.Cu") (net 7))
 (segment (start 51.816 68.645) (end 53.086 68.645) (width 0.3) (layer "F.Cu") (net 7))
 (segment (start 51.816 68.645) (end 51.816 66.675) (width 0.3) (layer "F.Cu") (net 7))
 (segment (start 54.483 91.567) (end 66.421 91.567) (width 0.3) (layer "F.Cu") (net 7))
 (segment (start 67.945 90.043) (end 67.945 86.11) (width 0.3) (layer "F.Cu") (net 7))
 (via (at 51.689 88.773) (size 0.7) (drill 0.3) (layers "F.Cu" "B.Cu") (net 7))
 (via (at 51.816 66.675) (size 0.7) (drill 0.3) (layers "F.Cu" "B.Cu") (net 7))
 (segment (start 51.816 66.675) (end 51.816 88.646) (width 0.3) (layer "B.Cu") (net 7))
 (segment (start 51.816 88.646) (end 51.689 88.773) (width 0.3) (layer "B.Cu") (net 7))
 (segment (start 50.8 50.8) (end 50.8 55.88) (width 0.3) (layer "F.Cu") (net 16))
 (segment (start 48.006 77.47) (end 48.641 78.105) (width 0.3) (layer "F.Cu") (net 14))
 (segment (start 48.006 48.514) (end 48.006 77.47) (width 0.3) (layer "F.Cu") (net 14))
 (segment (start 53.086 74.569999) (end 53.086 73.595) (width 0.3) (layer "F.Cu") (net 14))
 (segment (start 48.641 78.105) (end 52.197 78.105) (width 0.3) (layer "F.Cu") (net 14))
 (segment (start 50.8 45.72) (end 48.006 48.514) (width 0.3) (layer "F.Cu") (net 14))
 (segment (start 52.197 75.458999) (end 53.086 74.569999) (width 0.3) (layer "F.Cu") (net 14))
 (segment (start 52.197 78.105) (end 52.197 75.458999) (width 0.3) (layer "F.Cu") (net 14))
 (segment (start 53.594 65.024) (end 48.641 65.024) (width 0.3) (layer "F.Cu") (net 15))
 (segment (start 48.641 50.419) (end 50.8 48.26) (width 0.3) (layer "F.Cu") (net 15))
 (segment (start 48.641 65.024) (end 48.641 50.419) (width 0.3) (layer "F.Cu") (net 15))
 (segment (start 54.356 65.786) (end 53.594 65.024) (width 0.3) (layer "F.Cu") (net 15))
 (segment (start 51.435 77.343) (end 51.181 77.597) (width 0.3) (layer "F.Cu") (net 15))
 (segment (start 48.895 77.597) (end 48.641 77.343) (width 0.3) (layer "F.Cu") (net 15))
 (segment (start 54.356 68.645) (end 54.356 65.786) (width 0.3) (layer "F.Cu") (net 15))
 (segment (start 51.181 77.597) (end 48.895 77.597) (width 0.3) (layer "F.Cu") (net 15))
 (segment (start 48.641 77.343) (end 48.641 65.024) (width 0.3) (layer "F.Cu") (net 15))
 (segment (start 51.435 76.073) (end 51.435 77.343) (width 0.3) (layer "F.Cu") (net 15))
 (segment (start 73.275 83.185) (end 73.275 75.867) (width 0.3) (layer "F.Cu") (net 1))
 (segment (start 73.275 75.867) (end 61.976 64.568) (width 0.3) (layer "F.Cu") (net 1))
 (segment (start 50.206331 83.36334) (end 60.704671 72.865) (width 0.3) (layer "F.Cu") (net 5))
 (segment (start 60.704671 72.865) (end 61.976 72.865) (width 0.3) (layer "F.Cu") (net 5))
 (segment (start 53.4 83.57) (end 53.34 83.51) (width 0.3) (layer "F.Cu") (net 12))
 (segment (start 53.34 83.51) (end 53.34 85.09) (width 0.3) (layer "F.Cu") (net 12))
 (segment (start 59.755 83.82) (end 56.765 83.82) (width 0.3) (layer "F.Cu") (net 12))
 (segment (start 56.515 83.57) (end 53.4 83.57) (width 0.3) (layer "F.Cu") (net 12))
 (segment (start 56.765 83.82) (end 56.515 83.57) (width 0.3) (layer "F.Cu") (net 12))
 (segment (start 70.64 83.51) (end 68.005 83.51) (width 0.3) (layer "F.Cu") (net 4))
 (segment (start 67.945 85.09) (end 67.945 83.57) (width 0.3) (layer "F.Cu") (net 4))
 (segment (start 67.945 83.57) (end 66.425 85.09) (width 0.3) (layer "F.Cu") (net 4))
 (segment (start 68.005 83.51) (end 67.945 83.57) (width 0.3) (layer "F.Cu") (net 4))
 (segment (start 66.425 85.09) (end 64.705 85.09) (width 0.3) (layer "F.Cu") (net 4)))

